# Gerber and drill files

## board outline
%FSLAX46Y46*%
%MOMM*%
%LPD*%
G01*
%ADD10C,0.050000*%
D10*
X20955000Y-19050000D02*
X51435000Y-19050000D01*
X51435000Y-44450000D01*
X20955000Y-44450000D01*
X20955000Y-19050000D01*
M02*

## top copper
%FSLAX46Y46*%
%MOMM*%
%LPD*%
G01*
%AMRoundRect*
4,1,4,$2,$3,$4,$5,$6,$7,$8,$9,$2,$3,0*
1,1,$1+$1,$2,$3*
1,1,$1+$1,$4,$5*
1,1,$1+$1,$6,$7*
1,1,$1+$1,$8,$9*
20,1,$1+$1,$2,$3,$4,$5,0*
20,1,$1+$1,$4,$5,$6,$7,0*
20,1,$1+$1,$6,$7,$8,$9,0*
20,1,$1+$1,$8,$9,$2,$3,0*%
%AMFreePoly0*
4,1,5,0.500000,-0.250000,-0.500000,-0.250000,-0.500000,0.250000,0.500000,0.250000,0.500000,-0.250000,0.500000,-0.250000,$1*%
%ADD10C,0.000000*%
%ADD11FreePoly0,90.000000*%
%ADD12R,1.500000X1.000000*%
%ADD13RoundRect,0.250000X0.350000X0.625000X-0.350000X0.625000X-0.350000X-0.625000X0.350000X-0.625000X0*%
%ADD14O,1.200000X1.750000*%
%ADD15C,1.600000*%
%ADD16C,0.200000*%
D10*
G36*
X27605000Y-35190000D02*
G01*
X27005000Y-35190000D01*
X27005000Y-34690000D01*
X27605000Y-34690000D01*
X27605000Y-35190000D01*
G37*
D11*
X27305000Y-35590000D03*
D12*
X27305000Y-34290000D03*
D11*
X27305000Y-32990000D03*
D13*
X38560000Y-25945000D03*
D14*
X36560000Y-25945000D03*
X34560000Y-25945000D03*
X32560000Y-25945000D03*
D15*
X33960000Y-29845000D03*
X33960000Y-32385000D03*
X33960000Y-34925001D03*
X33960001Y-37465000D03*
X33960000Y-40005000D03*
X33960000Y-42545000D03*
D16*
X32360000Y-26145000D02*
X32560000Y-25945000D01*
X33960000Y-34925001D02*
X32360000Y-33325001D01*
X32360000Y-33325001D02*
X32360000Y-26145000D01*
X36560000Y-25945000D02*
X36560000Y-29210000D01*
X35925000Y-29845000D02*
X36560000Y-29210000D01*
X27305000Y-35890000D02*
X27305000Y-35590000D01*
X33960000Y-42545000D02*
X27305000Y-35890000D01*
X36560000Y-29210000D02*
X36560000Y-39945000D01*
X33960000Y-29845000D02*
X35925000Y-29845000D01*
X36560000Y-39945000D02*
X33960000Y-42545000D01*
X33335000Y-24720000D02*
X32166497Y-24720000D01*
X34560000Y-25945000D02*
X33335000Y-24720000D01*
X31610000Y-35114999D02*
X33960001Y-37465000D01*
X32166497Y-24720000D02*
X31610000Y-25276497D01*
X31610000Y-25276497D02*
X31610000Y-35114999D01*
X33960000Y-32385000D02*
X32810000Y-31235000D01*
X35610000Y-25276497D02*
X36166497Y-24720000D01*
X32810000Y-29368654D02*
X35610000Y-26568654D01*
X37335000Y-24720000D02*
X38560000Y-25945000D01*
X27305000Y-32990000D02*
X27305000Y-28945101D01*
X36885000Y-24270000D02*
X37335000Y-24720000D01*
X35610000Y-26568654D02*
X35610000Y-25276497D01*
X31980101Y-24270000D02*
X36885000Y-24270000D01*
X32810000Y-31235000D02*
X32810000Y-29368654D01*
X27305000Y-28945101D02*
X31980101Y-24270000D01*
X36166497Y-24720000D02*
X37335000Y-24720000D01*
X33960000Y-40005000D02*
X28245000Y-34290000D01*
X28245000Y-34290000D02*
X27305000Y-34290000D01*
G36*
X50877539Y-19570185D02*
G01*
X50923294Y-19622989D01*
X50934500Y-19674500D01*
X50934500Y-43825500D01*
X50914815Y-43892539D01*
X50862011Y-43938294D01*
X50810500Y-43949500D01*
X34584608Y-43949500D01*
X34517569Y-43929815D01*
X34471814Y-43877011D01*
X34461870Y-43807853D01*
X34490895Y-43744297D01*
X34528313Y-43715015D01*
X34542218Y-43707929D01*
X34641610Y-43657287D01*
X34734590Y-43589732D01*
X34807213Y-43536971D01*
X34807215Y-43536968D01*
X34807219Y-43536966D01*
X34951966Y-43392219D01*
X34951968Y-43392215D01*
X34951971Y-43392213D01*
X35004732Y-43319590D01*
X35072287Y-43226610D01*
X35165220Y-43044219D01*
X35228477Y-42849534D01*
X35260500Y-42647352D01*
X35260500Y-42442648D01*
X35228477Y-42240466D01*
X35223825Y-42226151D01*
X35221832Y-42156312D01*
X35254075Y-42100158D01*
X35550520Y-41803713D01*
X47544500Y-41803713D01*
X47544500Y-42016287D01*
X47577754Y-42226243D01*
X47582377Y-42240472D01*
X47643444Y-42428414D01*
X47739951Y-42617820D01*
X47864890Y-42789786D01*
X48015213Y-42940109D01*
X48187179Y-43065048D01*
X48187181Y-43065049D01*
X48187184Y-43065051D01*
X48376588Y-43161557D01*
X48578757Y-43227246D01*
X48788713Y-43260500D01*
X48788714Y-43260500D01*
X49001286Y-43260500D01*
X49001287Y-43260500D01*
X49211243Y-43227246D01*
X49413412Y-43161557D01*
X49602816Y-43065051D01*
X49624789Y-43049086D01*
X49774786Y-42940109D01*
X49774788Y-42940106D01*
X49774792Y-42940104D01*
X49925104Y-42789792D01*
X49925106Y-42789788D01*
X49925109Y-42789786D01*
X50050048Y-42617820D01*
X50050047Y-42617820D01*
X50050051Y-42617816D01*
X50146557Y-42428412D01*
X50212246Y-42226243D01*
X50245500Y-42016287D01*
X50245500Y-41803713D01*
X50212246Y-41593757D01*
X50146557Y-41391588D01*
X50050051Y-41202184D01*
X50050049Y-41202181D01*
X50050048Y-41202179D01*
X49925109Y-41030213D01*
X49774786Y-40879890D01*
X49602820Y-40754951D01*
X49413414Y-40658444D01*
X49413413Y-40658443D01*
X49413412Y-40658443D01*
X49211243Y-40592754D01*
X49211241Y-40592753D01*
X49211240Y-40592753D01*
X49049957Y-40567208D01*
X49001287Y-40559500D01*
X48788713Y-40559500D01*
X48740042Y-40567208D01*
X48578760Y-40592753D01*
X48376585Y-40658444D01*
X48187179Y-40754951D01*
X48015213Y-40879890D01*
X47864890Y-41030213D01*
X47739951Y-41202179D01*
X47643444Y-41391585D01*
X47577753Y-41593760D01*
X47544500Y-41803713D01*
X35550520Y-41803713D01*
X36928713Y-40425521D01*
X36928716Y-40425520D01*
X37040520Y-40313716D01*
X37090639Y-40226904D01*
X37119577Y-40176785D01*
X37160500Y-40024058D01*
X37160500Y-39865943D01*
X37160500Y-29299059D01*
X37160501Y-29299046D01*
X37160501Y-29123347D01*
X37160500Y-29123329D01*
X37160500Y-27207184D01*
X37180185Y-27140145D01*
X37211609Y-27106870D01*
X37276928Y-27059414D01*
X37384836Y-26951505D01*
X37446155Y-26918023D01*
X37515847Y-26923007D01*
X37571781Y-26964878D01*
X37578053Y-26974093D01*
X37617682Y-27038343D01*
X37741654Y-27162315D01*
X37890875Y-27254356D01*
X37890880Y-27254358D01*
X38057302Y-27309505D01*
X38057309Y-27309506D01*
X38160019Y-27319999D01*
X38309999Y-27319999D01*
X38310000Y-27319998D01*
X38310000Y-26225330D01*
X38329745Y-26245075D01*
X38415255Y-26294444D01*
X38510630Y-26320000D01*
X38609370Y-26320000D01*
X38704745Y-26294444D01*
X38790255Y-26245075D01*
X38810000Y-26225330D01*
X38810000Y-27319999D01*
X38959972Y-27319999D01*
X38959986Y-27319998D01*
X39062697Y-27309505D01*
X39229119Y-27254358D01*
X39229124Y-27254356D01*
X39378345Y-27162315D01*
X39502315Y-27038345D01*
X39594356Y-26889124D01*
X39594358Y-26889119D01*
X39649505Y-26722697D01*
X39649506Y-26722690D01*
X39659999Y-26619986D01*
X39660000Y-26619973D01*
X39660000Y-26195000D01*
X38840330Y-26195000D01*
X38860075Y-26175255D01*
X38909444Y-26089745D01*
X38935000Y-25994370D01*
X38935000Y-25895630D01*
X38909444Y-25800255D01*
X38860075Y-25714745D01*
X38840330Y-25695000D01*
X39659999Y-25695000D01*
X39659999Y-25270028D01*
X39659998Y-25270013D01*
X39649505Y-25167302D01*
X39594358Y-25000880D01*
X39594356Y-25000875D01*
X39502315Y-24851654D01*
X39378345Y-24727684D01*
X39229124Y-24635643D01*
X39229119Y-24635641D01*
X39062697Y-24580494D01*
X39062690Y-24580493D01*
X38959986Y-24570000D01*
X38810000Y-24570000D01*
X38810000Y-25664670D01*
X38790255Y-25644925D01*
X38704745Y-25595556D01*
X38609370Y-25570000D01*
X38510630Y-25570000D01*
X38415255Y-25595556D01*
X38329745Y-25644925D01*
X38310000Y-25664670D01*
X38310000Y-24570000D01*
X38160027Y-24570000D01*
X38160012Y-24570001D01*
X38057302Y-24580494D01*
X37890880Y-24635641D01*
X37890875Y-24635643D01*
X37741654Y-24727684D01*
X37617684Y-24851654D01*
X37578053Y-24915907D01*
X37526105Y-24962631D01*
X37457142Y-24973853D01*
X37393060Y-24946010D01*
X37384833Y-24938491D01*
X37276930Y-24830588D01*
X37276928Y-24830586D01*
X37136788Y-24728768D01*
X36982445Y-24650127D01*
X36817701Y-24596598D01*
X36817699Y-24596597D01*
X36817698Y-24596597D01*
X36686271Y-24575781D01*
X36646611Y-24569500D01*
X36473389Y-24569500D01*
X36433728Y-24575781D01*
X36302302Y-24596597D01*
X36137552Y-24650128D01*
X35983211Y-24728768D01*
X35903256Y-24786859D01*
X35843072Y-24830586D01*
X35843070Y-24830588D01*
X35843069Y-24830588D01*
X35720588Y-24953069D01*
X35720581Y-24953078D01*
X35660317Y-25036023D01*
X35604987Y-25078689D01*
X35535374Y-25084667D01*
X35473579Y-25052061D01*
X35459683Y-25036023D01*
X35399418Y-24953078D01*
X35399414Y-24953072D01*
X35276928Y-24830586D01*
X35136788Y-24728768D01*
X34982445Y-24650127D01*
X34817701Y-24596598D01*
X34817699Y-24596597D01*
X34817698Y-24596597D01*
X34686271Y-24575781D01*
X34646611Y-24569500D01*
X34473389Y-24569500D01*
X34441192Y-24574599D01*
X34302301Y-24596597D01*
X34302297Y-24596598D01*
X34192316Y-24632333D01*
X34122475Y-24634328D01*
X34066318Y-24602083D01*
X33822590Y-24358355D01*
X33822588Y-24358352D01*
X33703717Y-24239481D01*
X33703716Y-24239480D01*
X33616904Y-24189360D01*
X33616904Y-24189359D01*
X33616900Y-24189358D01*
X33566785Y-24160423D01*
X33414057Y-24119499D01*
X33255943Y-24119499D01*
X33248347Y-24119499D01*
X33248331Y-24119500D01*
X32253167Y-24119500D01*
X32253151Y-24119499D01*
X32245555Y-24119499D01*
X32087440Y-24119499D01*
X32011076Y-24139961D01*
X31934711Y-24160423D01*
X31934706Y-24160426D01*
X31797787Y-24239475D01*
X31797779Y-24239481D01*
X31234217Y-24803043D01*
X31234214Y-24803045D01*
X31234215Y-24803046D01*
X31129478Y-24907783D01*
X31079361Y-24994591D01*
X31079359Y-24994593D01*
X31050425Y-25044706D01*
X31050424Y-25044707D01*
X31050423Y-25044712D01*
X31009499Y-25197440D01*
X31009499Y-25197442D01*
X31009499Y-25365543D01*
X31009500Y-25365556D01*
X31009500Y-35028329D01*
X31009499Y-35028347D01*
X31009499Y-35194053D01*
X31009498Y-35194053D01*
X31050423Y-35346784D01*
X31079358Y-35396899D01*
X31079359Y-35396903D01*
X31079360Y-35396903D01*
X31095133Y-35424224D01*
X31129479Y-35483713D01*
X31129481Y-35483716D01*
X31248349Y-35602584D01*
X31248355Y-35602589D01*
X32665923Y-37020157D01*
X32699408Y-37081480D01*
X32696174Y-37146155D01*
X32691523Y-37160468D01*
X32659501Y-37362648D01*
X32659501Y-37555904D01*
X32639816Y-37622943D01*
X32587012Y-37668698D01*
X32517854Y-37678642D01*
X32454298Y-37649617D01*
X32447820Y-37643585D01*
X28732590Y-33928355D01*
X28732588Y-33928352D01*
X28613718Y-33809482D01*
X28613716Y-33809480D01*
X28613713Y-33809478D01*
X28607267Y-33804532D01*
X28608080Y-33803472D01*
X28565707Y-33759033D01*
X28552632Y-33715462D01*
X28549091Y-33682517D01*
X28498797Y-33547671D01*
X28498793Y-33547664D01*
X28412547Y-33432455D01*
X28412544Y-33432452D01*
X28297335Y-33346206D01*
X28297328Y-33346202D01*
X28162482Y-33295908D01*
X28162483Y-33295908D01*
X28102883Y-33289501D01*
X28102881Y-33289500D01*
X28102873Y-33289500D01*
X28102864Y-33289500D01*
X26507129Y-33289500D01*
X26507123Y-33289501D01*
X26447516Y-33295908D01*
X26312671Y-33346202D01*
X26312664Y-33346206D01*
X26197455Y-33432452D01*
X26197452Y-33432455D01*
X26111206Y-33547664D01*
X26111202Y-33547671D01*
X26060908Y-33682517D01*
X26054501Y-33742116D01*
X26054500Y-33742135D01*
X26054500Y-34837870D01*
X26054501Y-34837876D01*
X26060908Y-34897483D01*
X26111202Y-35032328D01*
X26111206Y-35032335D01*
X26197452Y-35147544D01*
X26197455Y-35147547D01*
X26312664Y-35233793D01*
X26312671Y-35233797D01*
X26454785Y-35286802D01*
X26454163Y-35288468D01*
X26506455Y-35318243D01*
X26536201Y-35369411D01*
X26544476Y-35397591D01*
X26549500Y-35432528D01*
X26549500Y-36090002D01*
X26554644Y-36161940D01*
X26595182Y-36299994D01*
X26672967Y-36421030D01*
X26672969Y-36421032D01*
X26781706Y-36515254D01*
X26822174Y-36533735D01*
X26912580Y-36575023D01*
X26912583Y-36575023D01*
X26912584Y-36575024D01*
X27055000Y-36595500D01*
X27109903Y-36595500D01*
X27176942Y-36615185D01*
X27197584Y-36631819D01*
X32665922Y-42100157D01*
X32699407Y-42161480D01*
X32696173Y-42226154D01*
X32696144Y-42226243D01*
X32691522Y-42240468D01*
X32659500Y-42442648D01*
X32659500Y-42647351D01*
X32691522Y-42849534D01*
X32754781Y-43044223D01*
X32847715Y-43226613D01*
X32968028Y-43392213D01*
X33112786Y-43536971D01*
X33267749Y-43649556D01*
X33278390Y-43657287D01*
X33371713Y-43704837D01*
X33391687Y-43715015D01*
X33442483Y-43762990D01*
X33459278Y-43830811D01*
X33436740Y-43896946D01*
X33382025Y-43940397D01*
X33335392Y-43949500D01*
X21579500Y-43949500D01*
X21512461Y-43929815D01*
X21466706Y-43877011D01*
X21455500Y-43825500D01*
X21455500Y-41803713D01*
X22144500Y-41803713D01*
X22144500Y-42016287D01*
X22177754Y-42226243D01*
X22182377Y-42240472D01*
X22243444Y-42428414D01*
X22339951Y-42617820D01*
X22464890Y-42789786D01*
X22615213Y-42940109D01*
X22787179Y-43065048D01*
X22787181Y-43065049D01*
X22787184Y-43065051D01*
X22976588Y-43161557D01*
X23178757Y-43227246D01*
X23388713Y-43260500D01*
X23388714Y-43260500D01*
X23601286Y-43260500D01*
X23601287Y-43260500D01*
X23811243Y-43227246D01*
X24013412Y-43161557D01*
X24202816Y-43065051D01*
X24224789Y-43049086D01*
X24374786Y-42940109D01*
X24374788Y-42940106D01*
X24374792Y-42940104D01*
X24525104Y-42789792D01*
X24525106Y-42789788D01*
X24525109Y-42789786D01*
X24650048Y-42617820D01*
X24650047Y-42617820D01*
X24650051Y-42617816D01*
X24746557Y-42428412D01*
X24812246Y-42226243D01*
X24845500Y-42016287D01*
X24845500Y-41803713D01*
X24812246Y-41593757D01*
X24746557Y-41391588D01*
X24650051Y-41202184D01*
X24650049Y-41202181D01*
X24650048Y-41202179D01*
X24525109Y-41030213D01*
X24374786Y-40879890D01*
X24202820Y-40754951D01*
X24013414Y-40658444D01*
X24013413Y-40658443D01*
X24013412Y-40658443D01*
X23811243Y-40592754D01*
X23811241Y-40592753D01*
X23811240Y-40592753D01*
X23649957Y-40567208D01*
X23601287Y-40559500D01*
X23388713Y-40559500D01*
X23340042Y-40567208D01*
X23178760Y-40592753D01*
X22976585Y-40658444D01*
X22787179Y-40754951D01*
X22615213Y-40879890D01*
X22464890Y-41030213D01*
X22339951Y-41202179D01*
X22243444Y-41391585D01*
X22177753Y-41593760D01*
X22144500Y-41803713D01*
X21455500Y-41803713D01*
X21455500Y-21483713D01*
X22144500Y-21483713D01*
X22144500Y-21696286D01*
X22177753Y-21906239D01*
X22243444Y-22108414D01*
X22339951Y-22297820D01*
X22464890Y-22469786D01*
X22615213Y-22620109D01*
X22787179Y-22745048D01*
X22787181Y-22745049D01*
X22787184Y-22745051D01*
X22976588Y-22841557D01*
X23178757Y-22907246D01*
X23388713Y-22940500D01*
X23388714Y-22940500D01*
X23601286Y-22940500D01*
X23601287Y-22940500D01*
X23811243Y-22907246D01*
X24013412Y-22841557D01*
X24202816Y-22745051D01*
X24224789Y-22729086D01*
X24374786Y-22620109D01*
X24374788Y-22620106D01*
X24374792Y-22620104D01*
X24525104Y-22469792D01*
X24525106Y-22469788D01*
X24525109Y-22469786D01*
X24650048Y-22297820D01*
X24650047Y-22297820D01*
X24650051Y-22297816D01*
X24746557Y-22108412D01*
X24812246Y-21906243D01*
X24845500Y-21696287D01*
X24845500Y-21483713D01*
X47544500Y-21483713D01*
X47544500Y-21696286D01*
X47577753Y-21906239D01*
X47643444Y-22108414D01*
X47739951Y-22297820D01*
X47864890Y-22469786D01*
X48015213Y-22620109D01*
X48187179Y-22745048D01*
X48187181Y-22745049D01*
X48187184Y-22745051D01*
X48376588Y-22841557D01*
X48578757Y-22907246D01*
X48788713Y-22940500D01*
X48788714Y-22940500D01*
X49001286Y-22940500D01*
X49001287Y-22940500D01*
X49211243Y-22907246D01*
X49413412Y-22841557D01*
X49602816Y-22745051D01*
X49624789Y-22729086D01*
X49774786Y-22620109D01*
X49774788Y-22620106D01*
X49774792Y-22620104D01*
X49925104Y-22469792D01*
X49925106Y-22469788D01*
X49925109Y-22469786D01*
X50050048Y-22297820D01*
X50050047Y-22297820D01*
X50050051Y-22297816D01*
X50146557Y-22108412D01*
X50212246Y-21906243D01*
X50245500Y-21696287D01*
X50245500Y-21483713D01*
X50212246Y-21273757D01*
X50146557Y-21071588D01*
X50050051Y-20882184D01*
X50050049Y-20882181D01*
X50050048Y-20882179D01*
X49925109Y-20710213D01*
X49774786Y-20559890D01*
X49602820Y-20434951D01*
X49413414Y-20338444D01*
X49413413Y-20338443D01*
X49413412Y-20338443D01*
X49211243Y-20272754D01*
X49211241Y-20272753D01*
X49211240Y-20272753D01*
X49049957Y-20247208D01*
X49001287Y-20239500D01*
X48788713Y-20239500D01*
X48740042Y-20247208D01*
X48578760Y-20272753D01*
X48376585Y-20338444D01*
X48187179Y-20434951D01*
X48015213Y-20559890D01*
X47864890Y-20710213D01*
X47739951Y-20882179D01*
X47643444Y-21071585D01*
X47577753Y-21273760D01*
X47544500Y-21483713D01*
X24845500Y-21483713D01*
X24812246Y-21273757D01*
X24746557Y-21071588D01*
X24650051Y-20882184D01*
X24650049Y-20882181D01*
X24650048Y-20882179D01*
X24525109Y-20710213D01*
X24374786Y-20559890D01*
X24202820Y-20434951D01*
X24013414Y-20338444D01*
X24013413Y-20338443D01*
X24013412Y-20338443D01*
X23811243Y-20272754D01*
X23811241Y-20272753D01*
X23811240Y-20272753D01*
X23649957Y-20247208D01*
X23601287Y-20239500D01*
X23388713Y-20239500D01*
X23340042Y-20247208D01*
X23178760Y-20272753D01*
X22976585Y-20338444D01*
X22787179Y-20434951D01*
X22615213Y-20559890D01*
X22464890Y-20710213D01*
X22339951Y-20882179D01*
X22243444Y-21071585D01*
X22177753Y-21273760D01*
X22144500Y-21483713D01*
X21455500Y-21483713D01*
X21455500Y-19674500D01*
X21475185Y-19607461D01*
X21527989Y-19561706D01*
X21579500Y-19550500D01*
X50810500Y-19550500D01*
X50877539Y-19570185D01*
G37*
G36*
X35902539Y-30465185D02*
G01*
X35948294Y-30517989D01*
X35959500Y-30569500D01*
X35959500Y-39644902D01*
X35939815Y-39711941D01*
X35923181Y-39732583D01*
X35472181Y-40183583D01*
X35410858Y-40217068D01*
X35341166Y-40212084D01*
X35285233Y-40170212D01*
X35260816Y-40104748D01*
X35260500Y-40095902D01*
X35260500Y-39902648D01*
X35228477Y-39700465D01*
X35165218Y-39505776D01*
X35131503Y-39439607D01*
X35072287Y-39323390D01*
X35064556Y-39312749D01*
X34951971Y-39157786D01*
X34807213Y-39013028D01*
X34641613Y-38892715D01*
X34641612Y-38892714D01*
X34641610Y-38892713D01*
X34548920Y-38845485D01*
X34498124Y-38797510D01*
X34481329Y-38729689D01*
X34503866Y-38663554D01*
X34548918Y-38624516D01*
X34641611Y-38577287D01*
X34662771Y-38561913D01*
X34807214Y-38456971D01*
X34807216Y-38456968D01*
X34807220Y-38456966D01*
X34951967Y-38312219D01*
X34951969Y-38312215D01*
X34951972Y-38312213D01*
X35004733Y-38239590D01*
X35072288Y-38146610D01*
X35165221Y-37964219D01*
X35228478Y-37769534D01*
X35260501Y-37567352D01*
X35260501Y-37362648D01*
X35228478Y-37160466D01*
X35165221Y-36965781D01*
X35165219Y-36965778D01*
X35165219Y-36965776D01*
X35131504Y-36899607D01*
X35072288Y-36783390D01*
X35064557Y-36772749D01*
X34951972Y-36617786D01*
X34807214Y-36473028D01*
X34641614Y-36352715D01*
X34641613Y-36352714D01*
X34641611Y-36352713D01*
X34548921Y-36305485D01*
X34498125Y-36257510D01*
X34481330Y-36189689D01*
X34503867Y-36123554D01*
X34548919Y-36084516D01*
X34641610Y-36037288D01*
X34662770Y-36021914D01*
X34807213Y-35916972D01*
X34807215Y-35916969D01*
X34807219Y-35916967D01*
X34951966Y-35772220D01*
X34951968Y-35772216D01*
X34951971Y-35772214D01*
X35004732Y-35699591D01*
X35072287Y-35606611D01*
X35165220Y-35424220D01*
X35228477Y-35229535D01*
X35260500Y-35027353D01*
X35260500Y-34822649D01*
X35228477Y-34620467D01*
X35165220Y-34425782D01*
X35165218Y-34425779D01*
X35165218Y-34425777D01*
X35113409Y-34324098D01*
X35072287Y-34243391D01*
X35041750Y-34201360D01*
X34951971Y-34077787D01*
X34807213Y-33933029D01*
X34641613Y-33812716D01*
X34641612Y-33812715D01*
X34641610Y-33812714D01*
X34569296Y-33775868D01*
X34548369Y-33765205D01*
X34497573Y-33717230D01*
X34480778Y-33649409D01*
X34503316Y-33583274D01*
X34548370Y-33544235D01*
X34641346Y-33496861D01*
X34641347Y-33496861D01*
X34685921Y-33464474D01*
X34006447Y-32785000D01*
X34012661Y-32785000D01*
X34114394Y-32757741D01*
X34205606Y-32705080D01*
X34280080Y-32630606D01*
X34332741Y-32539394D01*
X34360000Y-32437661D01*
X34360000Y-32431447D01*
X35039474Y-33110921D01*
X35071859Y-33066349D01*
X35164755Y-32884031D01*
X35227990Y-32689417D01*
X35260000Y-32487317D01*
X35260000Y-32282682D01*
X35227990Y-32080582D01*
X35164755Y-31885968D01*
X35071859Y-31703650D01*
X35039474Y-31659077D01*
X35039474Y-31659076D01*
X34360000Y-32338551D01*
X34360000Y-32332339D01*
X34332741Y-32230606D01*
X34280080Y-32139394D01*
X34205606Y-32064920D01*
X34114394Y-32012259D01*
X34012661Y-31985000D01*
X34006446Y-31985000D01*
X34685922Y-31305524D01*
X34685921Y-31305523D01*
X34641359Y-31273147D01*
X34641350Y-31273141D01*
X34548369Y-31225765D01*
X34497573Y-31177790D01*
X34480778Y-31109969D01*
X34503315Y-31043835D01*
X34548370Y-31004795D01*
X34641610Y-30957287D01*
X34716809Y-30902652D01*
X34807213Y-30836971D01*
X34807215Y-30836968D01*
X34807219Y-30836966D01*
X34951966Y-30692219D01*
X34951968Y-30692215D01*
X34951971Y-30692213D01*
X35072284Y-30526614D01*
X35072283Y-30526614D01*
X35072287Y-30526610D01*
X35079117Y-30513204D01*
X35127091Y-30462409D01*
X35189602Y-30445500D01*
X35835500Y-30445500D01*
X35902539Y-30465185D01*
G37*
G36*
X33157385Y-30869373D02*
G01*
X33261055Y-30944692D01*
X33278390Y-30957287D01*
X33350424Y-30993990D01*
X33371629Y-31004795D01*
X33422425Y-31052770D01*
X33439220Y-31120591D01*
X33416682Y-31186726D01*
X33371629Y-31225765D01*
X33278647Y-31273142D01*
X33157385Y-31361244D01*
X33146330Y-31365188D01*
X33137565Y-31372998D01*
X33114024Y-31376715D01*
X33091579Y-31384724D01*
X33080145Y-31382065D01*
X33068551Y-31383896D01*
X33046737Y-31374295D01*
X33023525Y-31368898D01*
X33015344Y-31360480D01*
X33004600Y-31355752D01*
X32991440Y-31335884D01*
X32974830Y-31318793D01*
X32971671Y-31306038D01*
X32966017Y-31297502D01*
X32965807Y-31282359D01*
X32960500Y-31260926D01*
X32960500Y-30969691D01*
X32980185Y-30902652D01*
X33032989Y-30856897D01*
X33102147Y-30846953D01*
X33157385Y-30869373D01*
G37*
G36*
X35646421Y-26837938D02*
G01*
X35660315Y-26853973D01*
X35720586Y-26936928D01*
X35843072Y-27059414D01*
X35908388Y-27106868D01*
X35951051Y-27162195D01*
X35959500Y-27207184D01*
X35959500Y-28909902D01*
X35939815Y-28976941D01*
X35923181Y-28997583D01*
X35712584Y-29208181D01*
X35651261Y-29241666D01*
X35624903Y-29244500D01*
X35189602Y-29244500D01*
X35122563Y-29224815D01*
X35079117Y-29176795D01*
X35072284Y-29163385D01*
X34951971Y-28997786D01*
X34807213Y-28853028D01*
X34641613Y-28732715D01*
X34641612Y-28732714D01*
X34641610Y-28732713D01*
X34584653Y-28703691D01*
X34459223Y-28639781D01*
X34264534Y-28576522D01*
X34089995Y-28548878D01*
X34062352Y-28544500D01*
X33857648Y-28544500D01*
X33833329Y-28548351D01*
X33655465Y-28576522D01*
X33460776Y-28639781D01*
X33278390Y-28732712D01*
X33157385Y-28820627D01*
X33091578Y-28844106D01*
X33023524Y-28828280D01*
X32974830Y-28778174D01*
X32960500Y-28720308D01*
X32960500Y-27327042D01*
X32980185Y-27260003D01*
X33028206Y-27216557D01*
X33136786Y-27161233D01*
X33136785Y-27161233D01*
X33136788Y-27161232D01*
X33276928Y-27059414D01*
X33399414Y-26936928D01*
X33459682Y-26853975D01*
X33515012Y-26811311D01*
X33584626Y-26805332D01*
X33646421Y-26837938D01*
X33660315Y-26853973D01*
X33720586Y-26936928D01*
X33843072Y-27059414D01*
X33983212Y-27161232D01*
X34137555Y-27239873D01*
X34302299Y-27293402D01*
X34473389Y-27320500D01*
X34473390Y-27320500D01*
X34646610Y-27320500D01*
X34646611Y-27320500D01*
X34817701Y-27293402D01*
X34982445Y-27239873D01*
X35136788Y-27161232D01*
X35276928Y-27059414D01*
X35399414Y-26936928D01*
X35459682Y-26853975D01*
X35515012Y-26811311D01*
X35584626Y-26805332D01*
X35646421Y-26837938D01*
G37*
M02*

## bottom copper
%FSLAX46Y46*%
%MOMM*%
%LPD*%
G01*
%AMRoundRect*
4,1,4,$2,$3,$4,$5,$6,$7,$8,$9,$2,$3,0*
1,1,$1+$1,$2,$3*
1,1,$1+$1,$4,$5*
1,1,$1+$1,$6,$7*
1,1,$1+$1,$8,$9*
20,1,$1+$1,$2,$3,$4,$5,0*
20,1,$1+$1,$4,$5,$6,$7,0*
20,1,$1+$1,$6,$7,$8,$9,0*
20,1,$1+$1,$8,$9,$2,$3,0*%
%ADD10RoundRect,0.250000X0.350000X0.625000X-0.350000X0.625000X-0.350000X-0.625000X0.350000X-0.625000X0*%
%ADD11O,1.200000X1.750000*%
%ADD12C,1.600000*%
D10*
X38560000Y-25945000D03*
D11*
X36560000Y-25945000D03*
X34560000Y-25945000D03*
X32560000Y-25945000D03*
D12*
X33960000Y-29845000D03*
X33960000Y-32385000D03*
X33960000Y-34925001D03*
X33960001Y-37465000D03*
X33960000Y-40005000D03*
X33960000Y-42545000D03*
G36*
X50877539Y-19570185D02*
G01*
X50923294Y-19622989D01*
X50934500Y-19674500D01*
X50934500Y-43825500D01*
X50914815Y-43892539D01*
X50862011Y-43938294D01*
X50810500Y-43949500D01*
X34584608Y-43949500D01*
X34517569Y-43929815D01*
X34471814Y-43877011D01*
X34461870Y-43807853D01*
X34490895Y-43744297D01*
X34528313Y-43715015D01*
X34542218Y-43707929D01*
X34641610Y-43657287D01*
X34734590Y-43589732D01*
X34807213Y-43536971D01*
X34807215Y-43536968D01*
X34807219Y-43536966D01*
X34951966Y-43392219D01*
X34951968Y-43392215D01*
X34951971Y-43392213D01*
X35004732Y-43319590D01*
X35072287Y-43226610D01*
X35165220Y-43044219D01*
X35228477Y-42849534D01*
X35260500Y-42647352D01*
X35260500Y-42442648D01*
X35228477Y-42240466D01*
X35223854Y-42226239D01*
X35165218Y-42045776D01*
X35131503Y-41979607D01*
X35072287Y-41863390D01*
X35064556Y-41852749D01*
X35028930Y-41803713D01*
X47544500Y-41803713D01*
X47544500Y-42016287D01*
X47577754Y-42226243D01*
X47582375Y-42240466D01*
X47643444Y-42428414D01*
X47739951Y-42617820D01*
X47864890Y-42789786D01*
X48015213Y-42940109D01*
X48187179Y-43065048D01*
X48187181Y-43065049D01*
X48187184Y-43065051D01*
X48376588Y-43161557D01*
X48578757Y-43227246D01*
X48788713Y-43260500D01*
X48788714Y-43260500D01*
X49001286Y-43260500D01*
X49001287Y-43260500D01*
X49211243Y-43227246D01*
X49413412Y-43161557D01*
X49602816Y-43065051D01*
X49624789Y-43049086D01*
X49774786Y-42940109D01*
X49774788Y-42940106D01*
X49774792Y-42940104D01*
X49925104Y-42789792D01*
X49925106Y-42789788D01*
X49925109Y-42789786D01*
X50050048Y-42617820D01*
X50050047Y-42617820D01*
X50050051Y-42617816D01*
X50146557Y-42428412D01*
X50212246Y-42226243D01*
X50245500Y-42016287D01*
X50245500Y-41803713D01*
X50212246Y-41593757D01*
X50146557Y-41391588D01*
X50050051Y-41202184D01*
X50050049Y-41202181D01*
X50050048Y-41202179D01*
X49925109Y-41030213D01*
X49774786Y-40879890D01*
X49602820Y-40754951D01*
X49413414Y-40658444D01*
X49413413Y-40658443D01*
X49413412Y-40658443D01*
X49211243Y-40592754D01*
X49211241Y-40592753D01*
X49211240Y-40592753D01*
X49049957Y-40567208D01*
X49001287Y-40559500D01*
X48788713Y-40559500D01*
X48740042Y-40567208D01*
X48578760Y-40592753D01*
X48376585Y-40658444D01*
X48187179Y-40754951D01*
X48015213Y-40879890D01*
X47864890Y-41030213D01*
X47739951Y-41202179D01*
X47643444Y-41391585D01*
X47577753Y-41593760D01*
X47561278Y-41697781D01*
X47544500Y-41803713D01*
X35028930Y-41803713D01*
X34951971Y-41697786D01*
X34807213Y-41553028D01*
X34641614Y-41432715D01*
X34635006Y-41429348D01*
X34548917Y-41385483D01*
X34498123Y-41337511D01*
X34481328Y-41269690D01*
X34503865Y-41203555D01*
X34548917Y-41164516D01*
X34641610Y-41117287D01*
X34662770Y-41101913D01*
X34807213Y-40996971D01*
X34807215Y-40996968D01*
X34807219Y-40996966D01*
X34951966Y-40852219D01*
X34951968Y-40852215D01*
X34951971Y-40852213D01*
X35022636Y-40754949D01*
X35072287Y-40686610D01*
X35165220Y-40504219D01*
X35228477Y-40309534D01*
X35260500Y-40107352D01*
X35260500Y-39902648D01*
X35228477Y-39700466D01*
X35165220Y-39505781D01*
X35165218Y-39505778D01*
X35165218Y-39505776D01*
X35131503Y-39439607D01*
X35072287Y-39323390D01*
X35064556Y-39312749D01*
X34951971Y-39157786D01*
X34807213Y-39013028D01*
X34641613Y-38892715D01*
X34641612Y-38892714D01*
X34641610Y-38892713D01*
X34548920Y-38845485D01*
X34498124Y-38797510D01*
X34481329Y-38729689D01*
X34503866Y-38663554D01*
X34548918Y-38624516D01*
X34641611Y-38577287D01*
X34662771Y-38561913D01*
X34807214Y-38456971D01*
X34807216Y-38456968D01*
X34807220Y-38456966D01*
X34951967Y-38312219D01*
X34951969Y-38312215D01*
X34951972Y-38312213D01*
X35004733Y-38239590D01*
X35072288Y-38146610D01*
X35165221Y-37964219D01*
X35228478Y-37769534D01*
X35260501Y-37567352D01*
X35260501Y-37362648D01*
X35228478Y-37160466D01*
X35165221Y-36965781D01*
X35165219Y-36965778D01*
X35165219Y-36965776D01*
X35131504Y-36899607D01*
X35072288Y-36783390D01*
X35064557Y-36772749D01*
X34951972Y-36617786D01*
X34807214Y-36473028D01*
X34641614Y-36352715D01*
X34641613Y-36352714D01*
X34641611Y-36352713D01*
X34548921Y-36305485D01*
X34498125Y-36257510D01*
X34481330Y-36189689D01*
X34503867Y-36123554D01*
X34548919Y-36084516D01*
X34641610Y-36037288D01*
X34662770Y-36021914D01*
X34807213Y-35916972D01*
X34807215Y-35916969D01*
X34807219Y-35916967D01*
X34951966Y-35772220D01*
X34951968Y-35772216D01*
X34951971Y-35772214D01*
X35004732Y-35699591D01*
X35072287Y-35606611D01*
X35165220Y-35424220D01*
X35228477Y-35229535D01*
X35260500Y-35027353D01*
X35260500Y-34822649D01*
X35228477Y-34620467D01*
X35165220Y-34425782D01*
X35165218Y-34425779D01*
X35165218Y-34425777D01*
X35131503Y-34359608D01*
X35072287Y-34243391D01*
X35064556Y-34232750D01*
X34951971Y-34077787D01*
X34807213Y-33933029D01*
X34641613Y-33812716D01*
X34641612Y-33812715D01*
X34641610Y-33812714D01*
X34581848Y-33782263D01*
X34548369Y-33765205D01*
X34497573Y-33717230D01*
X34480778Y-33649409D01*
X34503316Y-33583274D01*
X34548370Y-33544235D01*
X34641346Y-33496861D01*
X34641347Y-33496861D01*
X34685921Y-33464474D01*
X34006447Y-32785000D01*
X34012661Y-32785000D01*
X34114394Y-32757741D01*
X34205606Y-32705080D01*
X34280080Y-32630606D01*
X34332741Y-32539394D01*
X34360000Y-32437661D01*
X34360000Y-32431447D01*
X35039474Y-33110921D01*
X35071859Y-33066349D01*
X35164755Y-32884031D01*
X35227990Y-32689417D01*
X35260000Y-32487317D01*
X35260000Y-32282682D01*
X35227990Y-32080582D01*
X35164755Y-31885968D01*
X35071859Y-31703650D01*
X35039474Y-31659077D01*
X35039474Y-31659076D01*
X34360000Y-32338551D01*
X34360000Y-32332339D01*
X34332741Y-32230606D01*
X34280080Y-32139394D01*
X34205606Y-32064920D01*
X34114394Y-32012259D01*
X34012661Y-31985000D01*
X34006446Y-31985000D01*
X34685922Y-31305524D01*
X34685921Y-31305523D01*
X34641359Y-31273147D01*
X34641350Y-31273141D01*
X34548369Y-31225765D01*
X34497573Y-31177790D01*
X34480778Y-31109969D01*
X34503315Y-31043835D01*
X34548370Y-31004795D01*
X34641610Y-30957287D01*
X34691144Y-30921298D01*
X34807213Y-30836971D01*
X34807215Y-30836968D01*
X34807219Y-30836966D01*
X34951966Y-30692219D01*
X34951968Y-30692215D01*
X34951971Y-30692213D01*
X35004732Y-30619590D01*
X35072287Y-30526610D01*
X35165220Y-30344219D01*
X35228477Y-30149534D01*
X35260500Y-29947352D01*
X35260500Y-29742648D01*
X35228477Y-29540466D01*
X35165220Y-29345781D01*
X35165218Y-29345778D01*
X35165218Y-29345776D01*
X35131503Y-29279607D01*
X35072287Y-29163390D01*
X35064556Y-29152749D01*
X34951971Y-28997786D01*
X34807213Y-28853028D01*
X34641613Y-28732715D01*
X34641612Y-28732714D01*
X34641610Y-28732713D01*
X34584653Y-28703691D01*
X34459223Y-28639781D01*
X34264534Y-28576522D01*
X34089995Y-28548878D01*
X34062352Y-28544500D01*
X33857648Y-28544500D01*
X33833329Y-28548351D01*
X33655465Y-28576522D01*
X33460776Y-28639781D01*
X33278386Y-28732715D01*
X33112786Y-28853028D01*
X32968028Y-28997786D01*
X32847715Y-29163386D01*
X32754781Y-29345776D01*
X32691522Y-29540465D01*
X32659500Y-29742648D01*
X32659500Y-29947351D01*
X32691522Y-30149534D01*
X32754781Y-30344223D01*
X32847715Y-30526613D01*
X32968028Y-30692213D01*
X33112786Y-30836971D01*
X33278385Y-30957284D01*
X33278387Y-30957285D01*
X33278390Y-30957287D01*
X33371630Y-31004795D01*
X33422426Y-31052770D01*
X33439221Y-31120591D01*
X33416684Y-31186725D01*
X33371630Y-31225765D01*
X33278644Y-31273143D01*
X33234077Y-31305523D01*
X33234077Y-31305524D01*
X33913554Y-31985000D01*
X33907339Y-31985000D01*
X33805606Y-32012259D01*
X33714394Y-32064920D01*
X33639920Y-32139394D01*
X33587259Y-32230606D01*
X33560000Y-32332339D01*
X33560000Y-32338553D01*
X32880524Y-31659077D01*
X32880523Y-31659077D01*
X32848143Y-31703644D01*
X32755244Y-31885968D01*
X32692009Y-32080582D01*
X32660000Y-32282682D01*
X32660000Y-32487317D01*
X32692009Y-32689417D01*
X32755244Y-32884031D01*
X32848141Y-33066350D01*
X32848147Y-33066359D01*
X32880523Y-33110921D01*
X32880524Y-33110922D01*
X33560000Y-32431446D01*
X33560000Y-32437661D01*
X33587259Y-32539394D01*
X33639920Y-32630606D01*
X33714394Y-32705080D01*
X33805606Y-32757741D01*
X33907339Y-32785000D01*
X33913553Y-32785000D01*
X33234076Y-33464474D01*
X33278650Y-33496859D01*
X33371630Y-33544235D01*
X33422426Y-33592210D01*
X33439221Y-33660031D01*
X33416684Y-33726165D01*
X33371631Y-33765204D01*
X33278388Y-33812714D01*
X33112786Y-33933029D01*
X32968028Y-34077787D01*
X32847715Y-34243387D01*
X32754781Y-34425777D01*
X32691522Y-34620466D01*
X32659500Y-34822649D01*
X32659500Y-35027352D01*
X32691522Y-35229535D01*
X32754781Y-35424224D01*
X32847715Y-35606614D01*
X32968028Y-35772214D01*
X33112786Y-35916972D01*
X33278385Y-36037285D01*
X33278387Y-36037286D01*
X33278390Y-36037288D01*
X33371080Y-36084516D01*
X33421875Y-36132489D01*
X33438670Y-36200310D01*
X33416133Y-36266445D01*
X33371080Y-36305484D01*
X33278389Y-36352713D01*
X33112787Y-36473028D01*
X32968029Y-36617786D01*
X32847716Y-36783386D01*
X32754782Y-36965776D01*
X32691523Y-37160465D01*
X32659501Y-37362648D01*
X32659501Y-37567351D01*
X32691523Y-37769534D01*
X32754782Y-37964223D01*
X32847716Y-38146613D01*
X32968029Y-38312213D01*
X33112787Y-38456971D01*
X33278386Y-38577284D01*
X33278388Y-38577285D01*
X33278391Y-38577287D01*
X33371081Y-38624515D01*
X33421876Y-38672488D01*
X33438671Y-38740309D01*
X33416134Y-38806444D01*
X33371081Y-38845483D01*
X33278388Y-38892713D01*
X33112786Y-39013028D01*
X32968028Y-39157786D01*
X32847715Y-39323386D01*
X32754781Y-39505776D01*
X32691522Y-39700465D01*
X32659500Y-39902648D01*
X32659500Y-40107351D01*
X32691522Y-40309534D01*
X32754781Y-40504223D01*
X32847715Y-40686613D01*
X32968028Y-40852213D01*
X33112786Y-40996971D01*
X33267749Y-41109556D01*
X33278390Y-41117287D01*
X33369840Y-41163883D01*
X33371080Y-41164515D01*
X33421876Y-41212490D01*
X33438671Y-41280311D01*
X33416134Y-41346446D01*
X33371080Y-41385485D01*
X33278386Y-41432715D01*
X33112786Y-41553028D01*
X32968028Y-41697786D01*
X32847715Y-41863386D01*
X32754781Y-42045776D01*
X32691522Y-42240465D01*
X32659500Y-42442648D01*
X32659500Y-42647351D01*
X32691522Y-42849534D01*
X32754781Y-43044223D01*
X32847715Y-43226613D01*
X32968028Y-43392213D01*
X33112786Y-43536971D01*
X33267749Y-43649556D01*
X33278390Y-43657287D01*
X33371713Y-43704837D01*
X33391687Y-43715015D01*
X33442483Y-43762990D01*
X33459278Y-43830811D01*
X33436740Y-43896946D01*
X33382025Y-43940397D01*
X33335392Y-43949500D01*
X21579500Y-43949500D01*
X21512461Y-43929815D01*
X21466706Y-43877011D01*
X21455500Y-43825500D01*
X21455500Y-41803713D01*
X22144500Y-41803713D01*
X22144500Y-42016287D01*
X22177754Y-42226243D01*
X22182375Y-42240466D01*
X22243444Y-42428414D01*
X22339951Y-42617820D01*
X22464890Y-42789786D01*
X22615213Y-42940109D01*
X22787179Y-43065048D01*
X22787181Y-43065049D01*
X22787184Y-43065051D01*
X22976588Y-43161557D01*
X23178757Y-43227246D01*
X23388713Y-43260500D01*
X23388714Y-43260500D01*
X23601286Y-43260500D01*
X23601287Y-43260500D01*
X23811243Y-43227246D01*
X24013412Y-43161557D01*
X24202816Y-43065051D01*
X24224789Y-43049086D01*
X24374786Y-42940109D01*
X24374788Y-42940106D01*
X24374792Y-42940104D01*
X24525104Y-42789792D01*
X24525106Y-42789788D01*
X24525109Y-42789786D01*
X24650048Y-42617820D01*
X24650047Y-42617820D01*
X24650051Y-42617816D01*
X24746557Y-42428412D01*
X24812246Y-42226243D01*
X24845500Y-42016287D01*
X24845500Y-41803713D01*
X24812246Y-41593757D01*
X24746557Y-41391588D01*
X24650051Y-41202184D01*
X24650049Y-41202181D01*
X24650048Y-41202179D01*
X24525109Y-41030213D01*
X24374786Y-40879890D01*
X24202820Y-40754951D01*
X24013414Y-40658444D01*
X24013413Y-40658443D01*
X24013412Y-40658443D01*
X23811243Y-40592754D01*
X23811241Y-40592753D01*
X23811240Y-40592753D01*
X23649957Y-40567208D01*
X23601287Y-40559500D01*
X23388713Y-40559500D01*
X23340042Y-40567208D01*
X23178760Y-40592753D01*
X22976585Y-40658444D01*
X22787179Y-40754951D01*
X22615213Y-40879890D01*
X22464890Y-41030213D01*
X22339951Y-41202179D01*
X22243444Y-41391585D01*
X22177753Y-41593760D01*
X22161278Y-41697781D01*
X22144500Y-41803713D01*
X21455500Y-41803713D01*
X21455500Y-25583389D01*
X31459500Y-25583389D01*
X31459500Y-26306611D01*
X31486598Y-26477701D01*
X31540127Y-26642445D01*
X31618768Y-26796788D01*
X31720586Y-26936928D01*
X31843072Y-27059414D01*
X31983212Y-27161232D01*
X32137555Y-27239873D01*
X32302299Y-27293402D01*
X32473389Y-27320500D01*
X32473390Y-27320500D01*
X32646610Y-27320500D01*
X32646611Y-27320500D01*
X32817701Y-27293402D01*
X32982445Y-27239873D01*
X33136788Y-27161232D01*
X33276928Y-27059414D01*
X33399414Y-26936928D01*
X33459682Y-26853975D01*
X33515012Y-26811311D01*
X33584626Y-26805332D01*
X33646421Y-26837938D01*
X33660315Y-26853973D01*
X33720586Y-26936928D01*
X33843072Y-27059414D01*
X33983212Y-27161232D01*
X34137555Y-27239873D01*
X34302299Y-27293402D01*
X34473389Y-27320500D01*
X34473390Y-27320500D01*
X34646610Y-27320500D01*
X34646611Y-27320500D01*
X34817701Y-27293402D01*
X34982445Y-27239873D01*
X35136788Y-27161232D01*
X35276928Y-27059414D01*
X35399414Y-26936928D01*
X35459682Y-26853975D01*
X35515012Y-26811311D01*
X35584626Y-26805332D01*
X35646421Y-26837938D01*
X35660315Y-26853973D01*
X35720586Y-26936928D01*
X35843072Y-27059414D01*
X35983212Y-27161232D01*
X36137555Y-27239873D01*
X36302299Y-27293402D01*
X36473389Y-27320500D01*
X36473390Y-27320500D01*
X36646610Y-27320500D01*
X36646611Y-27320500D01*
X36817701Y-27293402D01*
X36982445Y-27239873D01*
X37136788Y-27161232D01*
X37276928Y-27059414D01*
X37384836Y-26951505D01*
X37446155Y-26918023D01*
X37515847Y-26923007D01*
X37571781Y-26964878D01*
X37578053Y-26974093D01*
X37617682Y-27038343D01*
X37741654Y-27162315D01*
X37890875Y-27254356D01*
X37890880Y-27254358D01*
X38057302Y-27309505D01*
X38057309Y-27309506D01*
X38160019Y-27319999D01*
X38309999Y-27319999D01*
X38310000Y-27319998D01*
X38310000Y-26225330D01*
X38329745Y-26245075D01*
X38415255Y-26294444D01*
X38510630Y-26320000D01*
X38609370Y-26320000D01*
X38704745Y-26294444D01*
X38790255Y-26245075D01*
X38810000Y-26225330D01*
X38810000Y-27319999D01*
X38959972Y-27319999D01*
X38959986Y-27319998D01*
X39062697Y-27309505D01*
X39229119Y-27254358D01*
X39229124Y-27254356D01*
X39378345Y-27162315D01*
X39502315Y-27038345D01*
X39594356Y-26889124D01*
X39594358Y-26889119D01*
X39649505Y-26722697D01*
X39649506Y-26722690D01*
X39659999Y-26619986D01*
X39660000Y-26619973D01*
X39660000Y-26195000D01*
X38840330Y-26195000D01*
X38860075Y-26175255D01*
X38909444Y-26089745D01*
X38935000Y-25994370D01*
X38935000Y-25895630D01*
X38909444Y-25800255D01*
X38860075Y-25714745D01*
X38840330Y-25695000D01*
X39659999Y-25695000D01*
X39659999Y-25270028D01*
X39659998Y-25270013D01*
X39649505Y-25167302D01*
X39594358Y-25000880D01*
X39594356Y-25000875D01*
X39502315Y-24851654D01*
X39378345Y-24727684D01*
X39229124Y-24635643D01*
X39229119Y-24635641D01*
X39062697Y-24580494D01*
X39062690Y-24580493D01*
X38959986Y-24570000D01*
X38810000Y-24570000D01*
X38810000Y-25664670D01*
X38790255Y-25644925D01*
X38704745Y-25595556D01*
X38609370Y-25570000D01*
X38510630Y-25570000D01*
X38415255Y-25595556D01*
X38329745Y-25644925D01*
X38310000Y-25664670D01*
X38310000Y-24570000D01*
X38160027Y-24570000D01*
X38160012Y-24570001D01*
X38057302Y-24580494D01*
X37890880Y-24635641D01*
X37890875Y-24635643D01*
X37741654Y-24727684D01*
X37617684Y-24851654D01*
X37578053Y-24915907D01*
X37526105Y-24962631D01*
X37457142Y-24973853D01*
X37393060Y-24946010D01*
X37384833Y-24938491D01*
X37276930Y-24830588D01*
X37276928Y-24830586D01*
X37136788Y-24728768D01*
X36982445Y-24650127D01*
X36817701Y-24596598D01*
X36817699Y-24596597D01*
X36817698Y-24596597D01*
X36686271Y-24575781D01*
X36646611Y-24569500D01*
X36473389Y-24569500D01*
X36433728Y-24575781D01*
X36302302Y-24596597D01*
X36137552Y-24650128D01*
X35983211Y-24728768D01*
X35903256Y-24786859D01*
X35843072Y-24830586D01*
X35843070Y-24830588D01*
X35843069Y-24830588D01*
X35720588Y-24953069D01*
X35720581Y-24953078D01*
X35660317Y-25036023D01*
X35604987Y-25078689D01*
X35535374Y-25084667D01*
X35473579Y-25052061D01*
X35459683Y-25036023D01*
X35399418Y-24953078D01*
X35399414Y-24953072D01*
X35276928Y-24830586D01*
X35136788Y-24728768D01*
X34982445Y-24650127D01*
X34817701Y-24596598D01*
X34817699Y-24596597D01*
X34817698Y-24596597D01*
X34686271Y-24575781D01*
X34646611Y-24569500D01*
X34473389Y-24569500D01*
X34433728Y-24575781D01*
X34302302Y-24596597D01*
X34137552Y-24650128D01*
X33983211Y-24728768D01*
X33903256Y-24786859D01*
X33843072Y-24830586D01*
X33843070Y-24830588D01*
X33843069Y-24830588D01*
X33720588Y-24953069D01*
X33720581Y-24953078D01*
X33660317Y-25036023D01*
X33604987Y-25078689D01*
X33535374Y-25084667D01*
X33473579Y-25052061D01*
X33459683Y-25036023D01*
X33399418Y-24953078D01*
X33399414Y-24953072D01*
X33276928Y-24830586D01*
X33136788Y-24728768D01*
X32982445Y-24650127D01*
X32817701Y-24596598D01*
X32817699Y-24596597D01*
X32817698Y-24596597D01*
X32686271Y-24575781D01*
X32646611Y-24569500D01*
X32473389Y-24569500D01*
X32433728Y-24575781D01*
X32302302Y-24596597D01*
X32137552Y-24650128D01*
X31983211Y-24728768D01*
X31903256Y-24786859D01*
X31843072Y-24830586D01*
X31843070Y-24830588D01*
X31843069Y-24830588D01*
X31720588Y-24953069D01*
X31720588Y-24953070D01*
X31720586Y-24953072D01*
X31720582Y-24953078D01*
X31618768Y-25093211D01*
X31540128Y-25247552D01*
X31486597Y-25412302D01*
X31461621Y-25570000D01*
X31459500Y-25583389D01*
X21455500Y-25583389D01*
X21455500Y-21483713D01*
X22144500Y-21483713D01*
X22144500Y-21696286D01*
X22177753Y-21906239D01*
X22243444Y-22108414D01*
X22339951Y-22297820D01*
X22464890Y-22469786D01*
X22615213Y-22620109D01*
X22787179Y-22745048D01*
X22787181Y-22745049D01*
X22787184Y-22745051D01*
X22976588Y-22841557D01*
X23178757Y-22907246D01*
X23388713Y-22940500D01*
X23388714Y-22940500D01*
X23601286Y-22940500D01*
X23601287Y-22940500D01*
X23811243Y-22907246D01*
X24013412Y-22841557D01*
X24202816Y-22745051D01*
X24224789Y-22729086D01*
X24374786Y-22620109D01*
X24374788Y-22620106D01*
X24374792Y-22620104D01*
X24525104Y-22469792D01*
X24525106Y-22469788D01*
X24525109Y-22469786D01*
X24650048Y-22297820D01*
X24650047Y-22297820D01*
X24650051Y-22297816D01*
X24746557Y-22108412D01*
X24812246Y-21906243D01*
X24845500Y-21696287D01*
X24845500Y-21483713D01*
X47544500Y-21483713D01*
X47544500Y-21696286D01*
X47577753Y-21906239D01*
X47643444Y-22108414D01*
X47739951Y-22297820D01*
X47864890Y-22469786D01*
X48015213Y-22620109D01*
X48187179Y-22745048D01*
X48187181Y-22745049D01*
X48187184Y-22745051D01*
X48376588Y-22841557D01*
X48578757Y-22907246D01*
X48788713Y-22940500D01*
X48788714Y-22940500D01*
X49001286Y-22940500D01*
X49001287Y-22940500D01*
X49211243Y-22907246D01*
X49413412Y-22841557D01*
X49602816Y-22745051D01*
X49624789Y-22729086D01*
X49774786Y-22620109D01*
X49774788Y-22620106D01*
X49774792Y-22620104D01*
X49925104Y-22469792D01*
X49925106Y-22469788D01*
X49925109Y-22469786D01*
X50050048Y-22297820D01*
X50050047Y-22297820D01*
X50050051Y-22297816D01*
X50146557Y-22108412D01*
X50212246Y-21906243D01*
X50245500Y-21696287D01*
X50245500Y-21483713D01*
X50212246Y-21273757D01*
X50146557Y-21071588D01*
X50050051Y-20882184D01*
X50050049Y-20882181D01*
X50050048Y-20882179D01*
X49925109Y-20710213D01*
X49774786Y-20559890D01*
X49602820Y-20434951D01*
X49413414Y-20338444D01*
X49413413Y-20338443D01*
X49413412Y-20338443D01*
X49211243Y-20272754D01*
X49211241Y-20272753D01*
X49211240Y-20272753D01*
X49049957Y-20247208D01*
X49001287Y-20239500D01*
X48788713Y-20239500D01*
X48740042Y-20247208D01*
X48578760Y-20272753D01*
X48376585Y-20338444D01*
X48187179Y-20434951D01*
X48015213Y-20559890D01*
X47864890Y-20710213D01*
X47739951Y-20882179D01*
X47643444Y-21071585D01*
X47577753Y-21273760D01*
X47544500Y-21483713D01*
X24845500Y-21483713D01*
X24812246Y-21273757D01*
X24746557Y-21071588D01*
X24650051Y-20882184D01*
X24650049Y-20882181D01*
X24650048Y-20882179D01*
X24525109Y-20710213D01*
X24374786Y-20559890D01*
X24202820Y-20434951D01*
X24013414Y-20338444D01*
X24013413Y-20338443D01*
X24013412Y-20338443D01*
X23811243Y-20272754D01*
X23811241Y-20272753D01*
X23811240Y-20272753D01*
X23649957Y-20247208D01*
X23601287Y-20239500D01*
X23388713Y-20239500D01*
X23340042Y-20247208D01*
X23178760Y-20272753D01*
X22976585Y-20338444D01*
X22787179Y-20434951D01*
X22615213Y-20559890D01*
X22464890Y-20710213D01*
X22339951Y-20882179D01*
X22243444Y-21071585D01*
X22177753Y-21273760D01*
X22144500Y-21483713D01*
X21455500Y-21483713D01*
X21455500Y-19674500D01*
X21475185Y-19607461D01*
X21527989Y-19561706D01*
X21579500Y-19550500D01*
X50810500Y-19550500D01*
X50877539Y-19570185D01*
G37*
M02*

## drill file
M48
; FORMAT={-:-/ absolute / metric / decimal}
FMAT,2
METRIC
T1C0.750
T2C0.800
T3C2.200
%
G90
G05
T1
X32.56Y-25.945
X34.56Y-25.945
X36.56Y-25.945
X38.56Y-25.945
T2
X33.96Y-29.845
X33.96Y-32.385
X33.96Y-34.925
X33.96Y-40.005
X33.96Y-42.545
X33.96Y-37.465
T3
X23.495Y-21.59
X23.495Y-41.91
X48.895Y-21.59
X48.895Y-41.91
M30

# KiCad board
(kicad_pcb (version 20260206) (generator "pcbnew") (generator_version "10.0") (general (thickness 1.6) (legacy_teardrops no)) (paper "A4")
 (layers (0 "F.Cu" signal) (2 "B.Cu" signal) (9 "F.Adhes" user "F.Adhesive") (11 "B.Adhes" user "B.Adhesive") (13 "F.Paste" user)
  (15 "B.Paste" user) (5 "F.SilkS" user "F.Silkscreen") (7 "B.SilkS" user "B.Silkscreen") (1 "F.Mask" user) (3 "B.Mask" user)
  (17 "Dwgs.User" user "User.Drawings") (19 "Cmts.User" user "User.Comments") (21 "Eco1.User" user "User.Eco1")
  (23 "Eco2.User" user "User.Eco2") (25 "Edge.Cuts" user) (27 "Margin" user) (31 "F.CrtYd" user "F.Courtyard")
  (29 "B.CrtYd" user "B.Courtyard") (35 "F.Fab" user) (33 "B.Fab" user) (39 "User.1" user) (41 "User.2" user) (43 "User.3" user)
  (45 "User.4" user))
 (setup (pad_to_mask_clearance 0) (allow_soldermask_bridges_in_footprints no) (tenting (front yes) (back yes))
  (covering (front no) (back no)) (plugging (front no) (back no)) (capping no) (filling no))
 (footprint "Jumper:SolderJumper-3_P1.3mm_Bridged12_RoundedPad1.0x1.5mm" (layer "F.Cu") (at 27.305 34.29 90)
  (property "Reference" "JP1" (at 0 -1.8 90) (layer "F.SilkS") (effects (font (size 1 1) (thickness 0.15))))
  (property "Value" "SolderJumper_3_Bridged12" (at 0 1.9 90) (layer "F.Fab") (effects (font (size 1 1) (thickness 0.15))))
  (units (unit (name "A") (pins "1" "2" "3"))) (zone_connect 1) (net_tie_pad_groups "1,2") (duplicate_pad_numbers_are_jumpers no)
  (fp_poly (pts (xy -0.9 -0.3) (xy -0.4 -0.3) (xy -0.4 0.3) (xy -0.9 0.3)) (stroke (width 0) (type solid)) (fill yes) (layer "F.Cu"))
  (pad "1" smd custom (at -1.3 0 90) (size 1 0.5) (layers "F.Cu" "F.Mask") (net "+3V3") (zone_connect 2) (thermal_bridge_angle 45)
   (options (clearance outline) (anchor rect)) (primitives))
  (pad "2" smd rect (at 0 0 90) (size 1 1.5) (layers "F.Cu" "F.Mask") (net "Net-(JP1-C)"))
  (pad "3" smd custom (at 1.3 0 90) (size 1 0.5) (layers "F.Cu" "F.Mask") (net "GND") (zone_connect 2) (thermal_bridge_angle 45)
   (options (clearance outline) (anchor rect)) (primitives)))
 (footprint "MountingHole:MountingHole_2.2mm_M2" (layer "F.Cu") (at 48.895 21.59)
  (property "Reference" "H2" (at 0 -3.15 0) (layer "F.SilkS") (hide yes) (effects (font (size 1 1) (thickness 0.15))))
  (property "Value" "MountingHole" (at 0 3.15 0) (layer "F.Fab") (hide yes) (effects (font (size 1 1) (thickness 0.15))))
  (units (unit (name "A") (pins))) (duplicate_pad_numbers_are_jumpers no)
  (pad "" np_thru_hole circle (at 0 0) (size 2.2 2.2) (drill 2.2) (layers "*.Cu" "*.Mask")))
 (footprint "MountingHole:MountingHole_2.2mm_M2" (layer "F.Cu") (at 48.895 41.91)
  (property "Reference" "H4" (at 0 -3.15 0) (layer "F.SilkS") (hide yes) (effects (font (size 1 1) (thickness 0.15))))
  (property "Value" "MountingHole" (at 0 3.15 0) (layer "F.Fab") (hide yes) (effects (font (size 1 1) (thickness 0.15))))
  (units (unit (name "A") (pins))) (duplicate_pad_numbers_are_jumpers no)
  (pad "" np_thru_hole circle (at 0 0) (size 2.2 2.2) (drill 2.2) (layers "*.Cu" "*.Mask")))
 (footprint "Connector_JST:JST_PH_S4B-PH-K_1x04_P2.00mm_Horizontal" (layer "F.Cu") (at 38.56 25.945 180)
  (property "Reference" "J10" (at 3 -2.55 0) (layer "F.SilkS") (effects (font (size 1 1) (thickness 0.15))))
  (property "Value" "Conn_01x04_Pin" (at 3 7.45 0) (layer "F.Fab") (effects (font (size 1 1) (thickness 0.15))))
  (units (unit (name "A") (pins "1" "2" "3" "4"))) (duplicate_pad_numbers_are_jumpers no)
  (pad "1" thru_hole roundrect (at 0 0 180) (size 1.2 1.75) (drill 0.75) (layers "*.Cu" "*.Mask") (remove_unused_layers no)
   (roundrect_rratio 0.208333) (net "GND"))
  (pad "2" thru_hole oval (at 2 0 180) (size 1.2 1.75) (drill 0.75) (layers "*.Cu" "*.Mask") (remove_unused_layers no) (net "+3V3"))
  (pad "3" thru_hole oval (at 4 0 180) (size 1.2 1.75) (drill 0.75) (layers "*.Cu" "*.Mask") (remove_unused_layers no) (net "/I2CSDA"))
  (pad "4" thru_hole oval (at 6 0 180) (size 1.2 1.75) (drill 0.75) (layers "*.Cu" "*.Mask") (remove_unused_layers no) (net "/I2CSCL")))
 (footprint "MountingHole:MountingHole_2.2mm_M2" (layer "F.Cu") (at 23.495 21.59)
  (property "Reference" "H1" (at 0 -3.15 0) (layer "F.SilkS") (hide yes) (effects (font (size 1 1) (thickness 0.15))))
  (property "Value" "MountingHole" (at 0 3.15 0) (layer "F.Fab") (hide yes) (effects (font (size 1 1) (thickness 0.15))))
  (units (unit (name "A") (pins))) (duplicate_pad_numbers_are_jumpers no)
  (pad "" np_thru_hole circle (at 0 0) (size 2.2 2.2) (drill 2.2) (layers "*.Cu" "*.Mask")))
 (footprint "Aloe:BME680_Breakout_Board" (layer "F.Cu") (at 40.31 36.195 -90)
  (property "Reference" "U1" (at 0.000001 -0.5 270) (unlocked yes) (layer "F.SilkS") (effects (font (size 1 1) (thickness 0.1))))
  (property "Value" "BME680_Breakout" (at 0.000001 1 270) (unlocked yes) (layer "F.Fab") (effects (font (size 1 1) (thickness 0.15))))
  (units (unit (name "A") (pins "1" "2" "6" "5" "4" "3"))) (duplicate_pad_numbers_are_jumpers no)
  (pad "1" thru_hole circle (at -6.35 6.35 270) (size 1.6 1.6) (drill 0.8) (layers "*.Cu" "*.Mask") (remove_unused_layers no) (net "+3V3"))
  (pad "2" thru_hole circle (at -3.81 6.35 270) (size 1.6 1.6) (drill 0.8) (layers "*.Cu" "*.Mask") (remove_unused_layers no) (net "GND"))
  (pad "3" thru_hole circle (at -1.269999 6.35 270) (size 1.6 1.6) (drill 0.8) (layers "*.Cu" "*.Mask") (remove_unused_layers no)
   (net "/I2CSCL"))
  (pad "4" thru_hole circle (at 1.27 6.349999 270) (size 1.6 1.6) (drill 0.8) (layers "*.Cu" "*.Mask") (remove_unused_layers no)
   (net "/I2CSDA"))
  (pad "5" thru_hole circle (at 3.81 6.35 270) (size 1.6 1.6) (drill 0.8) (layers "*.Cu" "*.Mask") (remove_unused_layers no)
   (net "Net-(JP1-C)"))
  (pad "6" thru_hole circle (at 6.35 6.35 270) (size 1.6 1.6) (drill 0.8) (layers "*.Cu" "*.Mask") (remove_unused_layers no) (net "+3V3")))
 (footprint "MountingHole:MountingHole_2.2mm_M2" (layer "F.Cu") (at 23.495 41.91)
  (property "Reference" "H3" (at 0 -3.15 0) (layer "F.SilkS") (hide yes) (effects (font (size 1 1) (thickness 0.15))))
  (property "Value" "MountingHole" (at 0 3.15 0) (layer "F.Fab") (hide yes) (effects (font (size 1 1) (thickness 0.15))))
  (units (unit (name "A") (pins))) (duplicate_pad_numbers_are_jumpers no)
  (pad "" np_thru_hole circle (at 0 0) (size 2.2 2.2) (drill 2.2) (layers "*.Cu" "*.Mask")))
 (gr_rect (start 20.955 19.05) (end 51.435 44.45) (stroke (width 0.05) (type solid)) (fill no) (layer "Edge.Cuts"))
 (segment (start 32.36 26.145) (end 32.56 25.945) (width 0.2) (layer "F.Cu") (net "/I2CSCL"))
 (segment (start 33.96 34.925001) (end 32.36 33.325001) (width 0.2) (layer "F.Cu") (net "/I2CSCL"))
 (segment (start 32.36 33.325001) (end 32.36 26.145) (width 0.2) (layer "F.Cu") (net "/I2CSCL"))
 (segment (start 36.56 25.945) (end 36.56 29.21) (width 0.2) (layer "F.Cu") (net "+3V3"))
 (segment (start 35.925 29.845) (end 36.56 29.21) (width 0.2) (layer "F.Cu") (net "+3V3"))
 (segment (start 27.305 35.89) (end 27.305 35.59) (width 0.2) (layer "F.Cu") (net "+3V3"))
 (segment (start 33.96 42.545) (end 27.305 35.89) (width 0.2) (layer "F.Cu") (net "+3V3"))
 (segment (start 36.56 29.21) (end 36.56 39.945) (width 0.2) (layer "F.Cu") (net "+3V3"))
 (segment (start 33.96 29.845) (end 35.925 29.845) (width 0.2) (layer "F.Cu") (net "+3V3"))
 (segment (start 36.56 39.945) (end 33.96 42.545) (width 0.2) (layer "F.Cu") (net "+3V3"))
 (segment (start 33.335 24.72) (end 32.166497 24.72) (width 0.2) (layer "F.Cu") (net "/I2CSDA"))
 (segment (start 34.56 25.945) (end 33.335 24.72) (width 0.2) (layer "F.Cu") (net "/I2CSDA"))
 (segment (start 31.61 35.114999) (end 33.960001 37.465) (width 0.2) (layer "F.Cu") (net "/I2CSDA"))
 (segment (start 32.166497 24.72) (end 31.61 25.276497) (width 0.2) (layer "F.Cu") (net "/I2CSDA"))
 (segment (start 31.61 25.276497) (end 31.61 35.114999) (width 0.2) (layer "F.Cu") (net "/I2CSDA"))
 (segment (start 33.96 32.385) (end 32.81 31.235) (width 0.2) (layer "F.Cu") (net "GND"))
 (segment (start 35.61 25.276497) (end 36.166497 24.72) (width 0.2) (layer "F.Cu") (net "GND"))
 (segment (start 32.81 29.368654) (end 35.61 26.568654) (width 0.2) (layer "F.Cu") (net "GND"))
 (segment (start 37.335 24.72) (end 38.56 25.945) (width 0.2) (layer "F.Cu") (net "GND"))
 (segment (start 27.305 32.99) (end 27.305 28.945101) (width 0.2) (layer "F.Cu") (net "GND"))
 (segment (start 36.885 24.27) (end 37.335 24.72) (width 0.2) (layer "F.Cu") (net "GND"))
 (segment (start 35.61 26.568654) (end 35.61 25.276497) (width 0.2) (layer "F.Cu") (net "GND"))
 (segment (start 31.980101 24.27) (end 36.885 24.27) (width 0.2) (layer "F.Cu") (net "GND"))
 (segment (start 32.81 31.235) (end 32.81 29.368654) (width 0.2) (layer "F.Cu") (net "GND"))
 (segment (start 27.305 28.945101) (end 31.980101 24.27) (width 0.2) (layer "F.Cu") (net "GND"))
 (segment (start 36.166497 24.72) (end 37.335 24.72) (width 0.2) (layer "F.Cu") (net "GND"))
 (segment (start 33.96 40.005) (end 28.245 34.29) (width 0.2) (layer "F.Cu") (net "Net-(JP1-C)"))
 (segment (start 28.245 34.29) (end 27.305 34.29) (width 0.2) (layer "F.Cu") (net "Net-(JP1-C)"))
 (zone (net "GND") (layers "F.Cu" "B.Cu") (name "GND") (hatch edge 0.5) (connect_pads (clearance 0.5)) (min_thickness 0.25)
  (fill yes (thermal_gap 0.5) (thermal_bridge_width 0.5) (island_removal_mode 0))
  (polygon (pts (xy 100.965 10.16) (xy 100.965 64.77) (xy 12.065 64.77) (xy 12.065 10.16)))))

